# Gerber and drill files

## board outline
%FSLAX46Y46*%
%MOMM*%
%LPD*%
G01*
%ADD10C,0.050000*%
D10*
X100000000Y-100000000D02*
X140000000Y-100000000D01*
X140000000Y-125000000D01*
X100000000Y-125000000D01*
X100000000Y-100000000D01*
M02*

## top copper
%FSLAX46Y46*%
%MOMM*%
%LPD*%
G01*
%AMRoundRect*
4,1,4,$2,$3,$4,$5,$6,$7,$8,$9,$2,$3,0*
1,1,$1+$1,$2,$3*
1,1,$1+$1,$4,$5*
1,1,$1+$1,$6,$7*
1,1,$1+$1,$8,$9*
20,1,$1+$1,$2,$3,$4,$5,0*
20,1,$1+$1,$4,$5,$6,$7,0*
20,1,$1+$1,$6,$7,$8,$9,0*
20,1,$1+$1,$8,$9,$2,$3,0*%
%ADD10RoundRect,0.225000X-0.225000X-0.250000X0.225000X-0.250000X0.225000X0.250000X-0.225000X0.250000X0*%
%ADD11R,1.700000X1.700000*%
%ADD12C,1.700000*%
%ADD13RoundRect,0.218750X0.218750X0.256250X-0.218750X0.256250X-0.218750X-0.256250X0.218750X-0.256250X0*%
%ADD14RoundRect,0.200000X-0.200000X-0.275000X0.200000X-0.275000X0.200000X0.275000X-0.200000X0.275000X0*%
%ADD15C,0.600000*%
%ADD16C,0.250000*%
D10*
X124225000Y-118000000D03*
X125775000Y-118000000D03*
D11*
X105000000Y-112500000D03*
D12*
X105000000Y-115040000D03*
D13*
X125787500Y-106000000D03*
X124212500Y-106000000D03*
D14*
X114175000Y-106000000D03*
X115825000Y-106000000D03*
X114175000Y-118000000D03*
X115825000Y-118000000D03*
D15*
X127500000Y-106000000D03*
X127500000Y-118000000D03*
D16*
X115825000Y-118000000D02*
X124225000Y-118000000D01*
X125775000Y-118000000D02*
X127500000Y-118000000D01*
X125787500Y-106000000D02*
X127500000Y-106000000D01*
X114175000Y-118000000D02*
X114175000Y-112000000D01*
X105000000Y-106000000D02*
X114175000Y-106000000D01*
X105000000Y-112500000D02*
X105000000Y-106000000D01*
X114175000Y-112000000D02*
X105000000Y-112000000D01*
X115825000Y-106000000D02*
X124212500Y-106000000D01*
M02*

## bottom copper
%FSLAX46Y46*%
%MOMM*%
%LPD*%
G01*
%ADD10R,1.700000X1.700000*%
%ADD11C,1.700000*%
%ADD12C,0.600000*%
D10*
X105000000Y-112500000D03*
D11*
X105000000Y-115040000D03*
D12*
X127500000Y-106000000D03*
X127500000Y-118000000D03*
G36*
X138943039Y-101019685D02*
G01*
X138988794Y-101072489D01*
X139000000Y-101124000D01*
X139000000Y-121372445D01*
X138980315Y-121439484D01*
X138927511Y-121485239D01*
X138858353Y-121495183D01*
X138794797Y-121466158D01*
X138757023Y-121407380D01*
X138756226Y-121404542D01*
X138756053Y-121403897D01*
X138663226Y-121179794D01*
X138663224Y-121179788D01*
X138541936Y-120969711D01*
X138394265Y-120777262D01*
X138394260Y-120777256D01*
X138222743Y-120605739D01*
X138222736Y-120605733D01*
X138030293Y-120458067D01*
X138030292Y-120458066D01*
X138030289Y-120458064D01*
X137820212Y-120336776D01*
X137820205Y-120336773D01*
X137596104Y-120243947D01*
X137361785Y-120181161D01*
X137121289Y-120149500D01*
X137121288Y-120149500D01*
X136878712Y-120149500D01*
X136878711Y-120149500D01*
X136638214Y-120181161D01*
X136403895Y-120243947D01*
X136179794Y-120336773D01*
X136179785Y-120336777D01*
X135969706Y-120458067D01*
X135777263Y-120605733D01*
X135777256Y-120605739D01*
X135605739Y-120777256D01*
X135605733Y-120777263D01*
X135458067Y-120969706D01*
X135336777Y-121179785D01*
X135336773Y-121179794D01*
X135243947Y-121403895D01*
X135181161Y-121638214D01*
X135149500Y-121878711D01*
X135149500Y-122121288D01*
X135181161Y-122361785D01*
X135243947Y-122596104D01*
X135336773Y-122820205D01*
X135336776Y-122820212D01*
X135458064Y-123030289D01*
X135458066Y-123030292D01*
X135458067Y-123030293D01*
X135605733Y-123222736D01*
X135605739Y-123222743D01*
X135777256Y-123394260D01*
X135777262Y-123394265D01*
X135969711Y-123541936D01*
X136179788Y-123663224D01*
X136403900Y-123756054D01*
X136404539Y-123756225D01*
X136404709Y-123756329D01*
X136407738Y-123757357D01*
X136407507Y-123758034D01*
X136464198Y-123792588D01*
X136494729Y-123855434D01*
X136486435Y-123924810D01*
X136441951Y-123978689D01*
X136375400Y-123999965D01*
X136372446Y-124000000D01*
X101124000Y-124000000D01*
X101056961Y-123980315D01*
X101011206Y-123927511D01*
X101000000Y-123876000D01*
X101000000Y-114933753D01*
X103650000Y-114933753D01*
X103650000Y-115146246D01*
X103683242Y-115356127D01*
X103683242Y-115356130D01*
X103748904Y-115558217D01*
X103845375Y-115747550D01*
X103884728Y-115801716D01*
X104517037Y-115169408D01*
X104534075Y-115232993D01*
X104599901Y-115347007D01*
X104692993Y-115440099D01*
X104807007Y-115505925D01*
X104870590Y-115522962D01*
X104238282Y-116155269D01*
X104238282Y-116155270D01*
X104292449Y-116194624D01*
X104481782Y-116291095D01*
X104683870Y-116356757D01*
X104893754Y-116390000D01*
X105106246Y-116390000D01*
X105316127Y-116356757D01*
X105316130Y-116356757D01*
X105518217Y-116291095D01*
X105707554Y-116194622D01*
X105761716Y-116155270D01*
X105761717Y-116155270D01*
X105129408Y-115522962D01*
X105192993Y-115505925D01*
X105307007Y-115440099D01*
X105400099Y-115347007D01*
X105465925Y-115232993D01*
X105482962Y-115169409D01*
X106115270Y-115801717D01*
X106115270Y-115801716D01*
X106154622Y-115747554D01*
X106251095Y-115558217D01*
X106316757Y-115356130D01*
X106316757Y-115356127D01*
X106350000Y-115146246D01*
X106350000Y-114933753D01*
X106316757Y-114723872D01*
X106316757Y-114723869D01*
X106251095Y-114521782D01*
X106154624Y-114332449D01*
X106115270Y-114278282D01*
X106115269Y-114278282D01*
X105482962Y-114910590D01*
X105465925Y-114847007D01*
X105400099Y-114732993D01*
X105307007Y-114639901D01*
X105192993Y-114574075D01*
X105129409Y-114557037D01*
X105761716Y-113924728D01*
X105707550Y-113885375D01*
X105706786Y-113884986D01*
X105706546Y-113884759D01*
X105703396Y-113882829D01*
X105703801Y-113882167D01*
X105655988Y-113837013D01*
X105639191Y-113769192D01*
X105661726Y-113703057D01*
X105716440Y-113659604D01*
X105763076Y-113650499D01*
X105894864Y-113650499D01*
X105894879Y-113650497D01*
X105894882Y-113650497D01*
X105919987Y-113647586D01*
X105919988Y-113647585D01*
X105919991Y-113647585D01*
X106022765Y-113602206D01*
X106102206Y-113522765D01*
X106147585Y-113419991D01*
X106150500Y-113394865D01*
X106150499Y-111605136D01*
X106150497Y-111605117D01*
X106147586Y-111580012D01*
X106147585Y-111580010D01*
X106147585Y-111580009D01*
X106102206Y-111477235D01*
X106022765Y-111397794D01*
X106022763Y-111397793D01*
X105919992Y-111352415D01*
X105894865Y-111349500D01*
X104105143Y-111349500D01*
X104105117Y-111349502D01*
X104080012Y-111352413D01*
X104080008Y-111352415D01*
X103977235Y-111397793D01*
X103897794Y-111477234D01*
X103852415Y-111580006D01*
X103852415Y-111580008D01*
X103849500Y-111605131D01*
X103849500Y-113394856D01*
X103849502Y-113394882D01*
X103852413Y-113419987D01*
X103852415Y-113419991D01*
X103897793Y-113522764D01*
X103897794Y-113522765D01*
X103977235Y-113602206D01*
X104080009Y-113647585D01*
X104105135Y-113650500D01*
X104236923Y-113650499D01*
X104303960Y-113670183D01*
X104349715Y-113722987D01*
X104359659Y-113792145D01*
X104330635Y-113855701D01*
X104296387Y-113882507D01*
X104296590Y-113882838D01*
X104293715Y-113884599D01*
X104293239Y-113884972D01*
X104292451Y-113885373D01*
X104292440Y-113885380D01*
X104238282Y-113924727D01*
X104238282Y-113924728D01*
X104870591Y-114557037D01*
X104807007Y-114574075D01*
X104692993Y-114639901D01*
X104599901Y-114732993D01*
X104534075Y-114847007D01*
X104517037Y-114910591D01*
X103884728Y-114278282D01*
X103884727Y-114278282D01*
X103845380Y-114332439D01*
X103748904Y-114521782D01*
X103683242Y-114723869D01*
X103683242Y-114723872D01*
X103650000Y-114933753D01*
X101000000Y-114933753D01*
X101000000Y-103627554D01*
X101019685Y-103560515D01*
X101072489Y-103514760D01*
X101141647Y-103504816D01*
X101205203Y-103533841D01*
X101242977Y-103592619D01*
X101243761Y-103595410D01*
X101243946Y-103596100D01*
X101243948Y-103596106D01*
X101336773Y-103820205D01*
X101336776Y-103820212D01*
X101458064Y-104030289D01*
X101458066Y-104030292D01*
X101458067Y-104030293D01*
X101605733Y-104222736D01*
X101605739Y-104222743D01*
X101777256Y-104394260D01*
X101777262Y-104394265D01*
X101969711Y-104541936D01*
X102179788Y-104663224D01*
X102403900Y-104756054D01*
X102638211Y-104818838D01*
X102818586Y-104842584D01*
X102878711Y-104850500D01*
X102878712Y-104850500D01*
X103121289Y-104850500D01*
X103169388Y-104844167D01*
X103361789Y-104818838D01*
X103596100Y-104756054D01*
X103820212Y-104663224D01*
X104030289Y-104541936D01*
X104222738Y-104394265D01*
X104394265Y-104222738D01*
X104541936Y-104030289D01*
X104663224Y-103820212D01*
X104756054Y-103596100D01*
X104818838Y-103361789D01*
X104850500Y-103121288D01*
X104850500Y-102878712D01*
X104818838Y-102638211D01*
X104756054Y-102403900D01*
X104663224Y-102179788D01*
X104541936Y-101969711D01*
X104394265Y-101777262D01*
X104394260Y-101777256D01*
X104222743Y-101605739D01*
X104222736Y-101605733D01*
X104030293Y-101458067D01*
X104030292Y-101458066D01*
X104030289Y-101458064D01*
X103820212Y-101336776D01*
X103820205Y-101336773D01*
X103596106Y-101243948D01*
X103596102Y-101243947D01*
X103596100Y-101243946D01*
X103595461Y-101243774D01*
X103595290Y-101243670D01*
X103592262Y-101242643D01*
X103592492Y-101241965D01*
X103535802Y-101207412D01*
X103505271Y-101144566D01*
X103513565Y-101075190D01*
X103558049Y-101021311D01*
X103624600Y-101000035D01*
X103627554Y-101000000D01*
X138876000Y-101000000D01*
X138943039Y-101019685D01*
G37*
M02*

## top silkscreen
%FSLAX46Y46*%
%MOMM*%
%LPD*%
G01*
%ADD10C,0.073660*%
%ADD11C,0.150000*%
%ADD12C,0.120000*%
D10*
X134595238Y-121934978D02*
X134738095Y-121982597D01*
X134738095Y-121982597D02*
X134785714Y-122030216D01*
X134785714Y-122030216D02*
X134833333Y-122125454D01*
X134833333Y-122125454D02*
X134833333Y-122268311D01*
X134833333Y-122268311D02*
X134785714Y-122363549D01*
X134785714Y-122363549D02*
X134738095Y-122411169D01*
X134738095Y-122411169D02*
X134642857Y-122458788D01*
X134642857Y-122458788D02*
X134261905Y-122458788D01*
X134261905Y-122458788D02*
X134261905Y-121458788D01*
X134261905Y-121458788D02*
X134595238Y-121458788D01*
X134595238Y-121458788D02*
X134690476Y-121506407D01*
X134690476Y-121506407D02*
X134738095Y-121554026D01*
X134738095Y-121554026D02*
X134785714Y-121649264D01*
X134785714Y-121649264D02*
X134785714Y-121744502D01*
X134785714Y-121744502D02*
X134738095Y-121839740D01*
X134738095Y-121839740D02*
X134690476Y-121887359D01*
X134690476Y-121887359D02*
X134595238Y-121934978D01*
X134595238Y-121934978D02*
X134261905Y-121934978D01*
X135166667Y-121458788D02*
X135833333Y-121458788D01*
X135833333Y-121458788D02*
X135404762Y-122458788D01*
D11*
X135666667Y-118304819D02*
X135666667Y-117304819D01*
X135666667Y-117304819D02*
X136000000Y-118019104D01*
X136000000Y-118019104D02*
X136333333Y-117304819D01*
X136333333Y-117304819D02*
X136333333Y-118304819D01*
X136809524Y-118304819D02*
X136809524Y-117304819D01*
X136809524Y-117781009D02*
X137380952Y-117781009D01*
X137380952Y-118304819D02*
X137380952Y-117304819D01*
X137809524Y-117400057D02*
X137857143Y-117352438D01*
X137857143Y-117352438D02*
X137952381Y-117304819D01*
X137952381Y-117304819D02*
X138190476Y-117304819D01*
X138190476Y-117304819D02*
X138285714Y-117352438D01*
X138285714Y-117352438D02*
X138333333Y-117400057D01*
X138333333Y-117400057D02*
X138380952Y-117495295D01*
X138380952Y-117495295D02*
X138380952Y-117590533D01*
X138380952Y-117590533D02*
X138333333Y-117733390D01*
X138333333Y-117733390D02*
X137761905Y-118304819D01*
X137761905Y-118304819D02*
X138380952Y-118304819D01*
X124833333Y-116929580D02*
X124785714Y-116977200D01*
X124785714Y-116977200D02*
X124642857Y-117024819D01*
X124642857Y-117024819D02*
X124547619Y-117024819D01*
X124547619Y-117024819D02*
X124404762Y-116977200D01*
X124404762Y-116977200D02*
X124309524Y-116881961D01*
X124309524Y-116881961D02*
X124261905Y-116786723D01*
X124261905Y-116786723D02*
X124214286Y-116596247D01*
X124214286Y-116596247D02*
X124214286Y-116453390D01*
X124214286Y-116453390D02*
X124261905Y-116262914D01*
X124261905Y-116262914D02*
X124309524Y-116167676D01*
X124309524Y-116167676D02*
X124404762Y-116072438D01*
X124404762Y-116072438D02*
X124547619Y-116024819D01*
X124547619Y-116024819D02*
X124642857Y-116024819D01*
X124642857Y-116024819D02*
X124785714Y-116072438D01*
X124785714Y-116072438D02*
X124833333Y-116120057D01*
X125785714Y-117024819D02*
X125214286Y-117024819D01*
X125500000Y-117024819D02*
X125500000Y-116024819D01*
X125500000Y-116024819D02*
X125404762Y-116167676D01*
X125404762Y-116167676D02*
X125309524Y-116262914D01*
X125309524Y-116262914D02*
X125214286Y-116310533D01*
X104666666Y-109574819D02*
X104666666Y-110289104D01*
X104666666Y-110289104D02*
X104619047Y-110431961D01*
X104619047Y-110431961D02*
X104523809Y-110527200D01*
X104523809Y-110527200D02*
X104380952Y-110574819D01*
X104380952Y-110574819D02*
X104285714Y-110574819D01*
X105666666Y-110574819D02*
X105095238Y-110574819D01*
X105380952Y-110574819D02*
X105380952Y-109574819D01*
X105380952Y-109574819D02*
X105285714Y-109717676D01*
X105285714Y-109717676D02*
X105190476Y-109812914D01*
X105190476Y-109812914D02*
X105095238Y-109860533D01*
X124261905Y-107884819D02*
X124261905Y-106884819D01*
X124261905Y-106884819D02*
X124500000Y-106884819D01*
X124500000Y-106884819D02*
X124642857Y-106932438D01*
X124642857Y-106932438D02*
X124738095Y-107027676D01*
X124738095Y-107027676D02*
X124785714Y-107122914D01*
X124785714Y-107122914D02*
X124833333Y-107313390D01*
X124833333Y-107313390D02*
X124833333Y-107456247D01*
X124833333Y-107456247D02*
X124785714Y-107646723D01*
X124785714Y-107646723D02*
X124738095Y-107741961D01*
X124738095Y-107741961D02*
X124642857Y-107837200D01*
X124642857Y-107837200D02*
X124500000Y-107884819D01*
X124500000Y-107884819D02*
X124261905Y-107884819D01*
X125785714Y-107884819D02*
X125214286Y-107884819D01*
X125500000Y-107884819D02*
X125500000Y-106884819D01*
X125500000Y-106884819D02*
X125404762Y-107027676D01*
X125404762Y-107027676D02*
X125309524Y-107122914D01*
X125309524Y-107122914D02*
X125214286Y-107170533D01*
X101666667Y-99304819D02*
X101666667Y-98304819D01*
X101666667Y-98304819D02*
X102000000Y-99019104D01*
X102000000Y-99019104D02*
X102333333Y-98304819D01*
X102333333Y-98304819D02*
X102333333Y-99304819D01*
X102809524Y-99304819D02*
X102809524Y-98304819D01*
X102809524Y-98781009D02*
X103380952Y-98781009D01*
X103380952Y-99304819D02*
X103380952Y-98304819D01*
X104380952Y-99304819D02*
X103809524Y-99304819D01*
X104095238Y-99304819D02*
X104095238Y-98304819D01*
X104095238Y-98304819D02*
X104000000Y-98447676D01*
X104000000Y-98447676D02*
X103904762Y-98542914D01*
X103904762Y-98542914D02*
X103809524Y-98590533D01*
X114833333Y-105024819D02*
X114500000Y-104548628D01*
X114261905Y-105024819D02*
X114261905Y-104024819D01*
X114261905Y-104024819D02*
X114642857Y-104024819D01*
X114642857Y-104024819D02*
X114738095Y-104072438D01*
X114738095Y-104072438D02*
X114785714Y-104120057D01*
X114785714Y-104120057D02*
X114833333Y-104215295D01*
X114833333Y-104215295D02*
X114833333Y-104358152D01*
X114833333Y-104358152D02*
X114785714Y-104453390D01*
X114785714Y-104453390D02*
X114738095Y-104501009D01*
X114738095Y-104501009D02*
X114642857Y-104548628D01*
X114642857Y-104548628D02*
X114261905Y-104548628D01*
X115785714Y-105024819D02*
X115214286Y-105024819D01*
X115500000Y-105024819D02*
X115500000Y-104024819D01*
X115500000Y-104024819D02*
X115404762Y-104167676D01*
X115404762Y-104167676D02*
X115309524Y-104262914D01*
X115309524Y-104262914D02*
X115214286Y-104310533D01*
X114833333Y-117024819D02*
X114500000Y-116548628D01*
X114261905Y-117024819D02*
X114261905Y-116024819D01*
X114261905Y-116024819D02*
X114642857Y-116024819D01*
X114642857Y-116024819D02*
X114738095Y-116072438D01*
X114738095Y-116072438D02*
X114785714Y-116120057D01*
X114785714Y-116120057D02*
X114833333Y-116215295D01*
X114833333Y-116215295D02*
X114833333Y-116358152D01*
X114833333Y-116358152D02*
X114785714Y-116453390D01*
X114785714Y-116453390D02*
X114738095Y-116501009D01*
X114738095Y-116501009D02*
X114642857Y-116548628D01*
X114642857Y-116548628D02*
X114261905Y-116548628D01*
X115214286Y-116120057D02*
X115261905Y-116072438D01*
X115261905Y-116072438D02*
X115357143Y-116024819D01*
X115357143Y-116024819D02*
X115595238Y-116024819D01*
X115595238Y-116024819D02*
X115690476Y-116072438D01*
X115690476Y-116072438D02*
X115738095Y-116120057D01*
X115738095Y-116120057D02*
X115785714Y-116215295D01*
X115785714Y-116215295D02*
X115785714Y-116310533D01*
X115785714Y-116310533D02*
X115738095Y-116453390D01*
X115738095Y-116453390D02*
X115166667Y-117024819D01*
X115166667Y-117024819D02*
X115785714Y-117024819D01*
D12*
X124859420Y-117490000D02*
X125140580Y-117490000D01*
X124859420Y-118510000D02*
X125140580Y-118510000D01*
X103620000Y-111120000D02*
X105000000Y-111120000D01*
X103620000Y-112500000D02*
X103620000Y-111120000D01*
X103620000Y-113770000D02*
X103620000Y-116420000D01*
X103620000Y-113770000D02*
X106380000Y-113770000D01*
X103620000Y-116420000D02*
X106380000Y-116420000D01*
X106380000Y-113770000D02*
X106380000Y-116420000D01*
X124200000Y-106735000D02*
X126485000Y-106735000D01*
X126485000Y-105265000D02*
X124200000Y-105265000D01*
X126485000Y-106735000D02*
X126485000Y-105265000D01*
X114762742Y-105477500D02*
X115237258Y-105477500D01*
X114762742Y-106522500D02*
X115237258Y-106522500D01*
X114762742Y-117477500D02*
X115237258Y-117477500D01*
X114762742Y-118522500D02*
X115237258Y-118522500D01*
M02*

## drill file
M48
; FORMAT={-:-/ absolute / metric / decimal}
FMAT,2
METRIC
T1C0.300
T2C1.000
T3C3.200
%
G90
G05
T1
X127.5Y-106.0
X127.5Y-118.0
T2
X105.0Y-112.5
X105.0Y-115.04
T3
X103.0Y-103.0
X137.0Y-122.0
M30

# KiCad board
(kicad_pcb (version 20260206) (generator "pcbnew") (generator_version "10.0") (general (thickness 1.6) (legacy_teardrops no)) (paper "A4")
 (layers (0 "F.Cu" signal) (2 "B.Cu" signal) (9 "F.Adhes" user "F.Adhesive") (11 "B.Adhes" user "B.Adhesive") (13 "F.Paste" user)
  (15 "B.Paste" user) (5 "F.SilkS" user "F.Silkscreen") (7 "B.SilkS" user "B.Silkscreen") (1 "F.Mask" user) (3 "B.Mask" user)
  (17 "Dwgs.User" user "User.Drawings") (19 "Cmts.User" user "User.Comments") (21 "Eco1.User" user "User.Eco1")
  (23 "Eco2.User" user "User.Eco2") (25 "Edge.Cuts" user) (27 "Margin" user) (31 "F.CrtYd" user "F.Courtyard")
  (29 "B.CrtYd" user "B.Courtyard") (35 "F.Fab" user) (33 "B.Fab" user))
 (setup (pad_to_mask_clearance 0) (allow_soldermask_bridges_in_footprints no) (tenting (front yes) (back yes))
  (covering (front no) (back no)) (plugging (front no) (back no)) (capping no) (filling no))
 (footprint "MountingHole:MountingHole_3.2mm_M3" (layer "F.Cu") (at 137 122)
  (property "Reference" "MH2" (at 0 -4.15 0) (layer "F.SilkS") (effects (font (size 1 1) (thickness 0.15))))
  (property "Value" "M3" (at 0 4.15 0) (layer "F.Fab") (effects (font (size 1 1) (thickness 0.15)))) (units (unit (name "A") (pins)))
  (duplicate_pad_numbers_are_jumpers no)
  (pad "" np_thru_hole circle (at 0 0) (size 3.2 3.2) (drill 3.2) (layers "*.Cu" "*.Mask")))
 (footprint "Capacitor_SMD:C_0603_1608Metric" (layer "F.Cu") (at 125 118)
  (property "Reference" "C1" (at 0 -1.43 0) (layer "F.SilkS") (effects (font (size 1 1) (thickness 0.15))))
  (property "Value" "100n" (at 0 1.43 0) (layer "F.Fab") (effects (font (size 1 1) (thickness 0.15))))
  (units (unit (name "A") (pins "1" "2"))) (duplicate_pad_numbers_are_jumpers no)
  (fp_line (start -0.14058 -0.51) (end 0.14058 -0.51) (stroke (width 0.12) (type solid)) (layer "F.SilkS"))
  (fp_line (start -0.14058 0.51) (end 0.14058 0.51) (stroke (width 0.12) (type solid)) (layer "F.SilkS"))
  (pad "1" smd roundrect (at -0.775 0) (size 0.9 0.95) (layers "F.Cu" "F.Mask" "F.Paste") (roundrect_rratio 0.25) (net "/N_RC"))
  (pad "2" smd roundrect (at 0.775 0) (size 0.9 0.95) (layers "F.Cu" "F.Mask" "F.Paste") (roundrect_rratio 0.25) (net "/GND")))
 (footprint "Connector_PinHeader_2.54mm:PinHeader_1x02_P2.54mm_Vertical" (layer "F.Cu") (at 105 112.5)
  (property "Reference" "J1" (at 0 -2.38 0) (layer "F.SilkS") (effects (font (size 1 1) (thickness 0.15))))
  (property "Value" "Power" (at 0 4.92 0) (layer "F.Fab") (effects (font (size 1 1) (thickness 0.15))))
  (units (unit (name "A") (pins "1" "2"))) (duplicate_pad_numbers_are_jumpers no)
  (fp_line (start -1.38 -1.38) (end 0 -1.38) (stroke (width 0.12) (type solid)) (layer "F.SilkS"))
  (fp_line (start -1.38 0) (end -1.38 -1.38) (stroke (width 0.12) (type solid)) (layer "F.SilkS"))
  (fp_line (start -1.38 1.27) (end -1.38 3.92) (stroke (width 0.12) (type solid)) (layer "F.SilkS"))
  (fp_line (start -1.38 1.27) (end 1.38 1.27) (stroke (width 0.12) (type solid)) (layer "F.SilkS"))
  (fp_line (start -1.38 3.92) (end 1.38 3.92) (stroke (width 0.12) (type solid)) (layer "F.SilkS"))
  (fp_line (start 1.38 1.27) (end 1.38 3.92) (stroke (width 0.12) (type solid)) (layer "F.SilkS"))
  (pad "1" thru_hole rect (at 0 0) (size 1.7 1.7) (drill 1) (layers "*.Cu" "*.Mask") (remove_unused_layers no) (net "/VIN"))
  (pad "2" thru_hole circle (at 0 2.54) (size 1.7 1.7) (drill 1) (layers "*.Cu" "*.Mask") (remove_unused_layers no) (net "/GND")))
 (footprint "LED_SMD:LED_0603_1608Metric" (layer "F.Cu") (at 125 106 180)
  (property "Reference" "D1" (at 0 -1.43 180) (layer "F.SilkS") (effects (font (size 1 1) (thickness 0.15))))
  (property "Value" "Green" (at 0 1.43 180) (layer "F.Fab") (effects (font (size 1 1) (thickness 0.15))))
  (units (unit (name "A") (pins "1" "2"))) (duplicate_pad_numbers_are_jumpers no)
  (fp_line (start 0.8 -0.735) (end -1.485 -0.735) (stroke (width 0.12) (type solid)) (layer "F.SilkS"))
  (fp_line (start -1.485 0.735) (end 0.8 0.735) (stroke (width 0.12) (type solid)) (layer "F.SilkS"))
  (fp_line (start -1.485 -0.735) (end -1.485 0.735) (stroke (width 0.12) (type solid)) (layer "F.SilkS"))
  (pad "1" smd roundrect (at -0.7875 0 180) (size 0.875 0.95) (layers "F.Cu" "F.Mask" "F.Paste") (roundrect_rratio 0.25) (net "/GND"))
  (pad "2" smd roundrect (at 0.7875 0 180) (size 0.875 0.95) (layers "F.Cu" "F.Mask" "F.Paste") (roundrect_rratio 0.25) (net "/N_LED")))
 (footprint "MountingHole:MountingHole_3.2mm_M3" (layer "F.Cu") (at 103 103)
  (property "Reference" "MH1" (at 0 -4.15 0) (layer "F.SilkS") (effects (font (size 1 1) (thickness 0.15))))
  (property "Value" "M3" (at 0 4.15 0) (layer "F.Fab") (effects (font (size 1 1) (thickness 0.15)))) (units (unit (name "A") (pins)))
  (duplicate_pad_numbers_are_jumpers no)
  (pad "" np_thru_hole circle (at 0 0) (size 3.2 3.2) (drill 3.2) (layers "*.Cu" "*.Mask")))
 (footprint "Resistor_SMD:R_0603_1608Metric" (layer "F.Cu") (at 115 106)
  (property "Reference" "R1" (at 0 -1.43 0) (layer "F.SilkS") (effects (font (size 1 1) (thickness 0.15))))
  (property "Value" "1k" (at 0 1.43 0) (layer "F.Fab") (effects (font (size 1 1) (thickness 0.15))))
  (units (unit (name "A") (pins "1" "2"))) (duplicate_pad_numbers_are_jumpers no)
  (fp_line (start -0.237258 -0.5225) (end 0.237258 -0.5225) (stroke (width 0.12) (type solid)) (layer "F.SilkS"))
  (fp_line (start -0.237258 0.5225) (end 0.237258 0.5225) (stroke (width 0.12) (type solid)) (layer "F.SilkS"))
  (pad "1" smd roundrect (at -0.825 0) (size 0.8 0.95) (layers "F.Cu" "F.Mask" "F.Paste") (roundrect_rratio 0.25) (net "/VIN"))
  (pad "2" smd roundrect (at 0.825 0) (size 0.8 0.95) (layers "F.Cu" "F.Mask" "F.Paste") (roundrect_rratio 0.25) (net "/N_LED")))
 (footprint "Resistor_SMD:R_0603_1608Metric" (layer "F.Cu") (at 115 118)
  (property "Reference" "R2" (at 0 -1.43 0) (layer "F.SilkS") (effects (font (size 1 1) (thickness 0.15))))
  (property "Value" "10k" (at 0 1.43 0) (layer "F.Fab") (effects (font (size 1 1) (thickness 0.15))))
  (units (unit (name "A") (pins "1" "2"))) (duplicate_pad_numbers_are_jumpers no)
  (fp_line (start -0.237258 -0.5225) (end 0.237258 -0.5225) (stroke (width 0.12) (type solid)) (layer "F.SilkS"))
  (fp_line (start -0.237258 0.5225) (end 0.237258 0.5225) (stroke (width 0.12) (type solid)) (layer "F.SilkS"))
  (pad "1" smd roundrect (at -0.825 0) (size 0.8 0.95) (layers "F.Cu" "F.Mask" "F.Paste") (roundrect_rratio 0.25) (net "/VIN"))
  (pad "2" smd roundrect (at 0.825 0) (size 0.8 0.95) (layers "F.Cu" "F.Mask" "F.Paste") (roundrect_rratio 0.25) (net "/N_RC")))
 (gr_rect (start 100 100) (end 140 125) (stroke (width 0.05) (type default)) (fill no) (layer "Edge.Cuts"))
 (segment (start 115.825 118) (end 124.225 118) (width 0.25) (layer "F.Cu") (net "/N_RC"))
 (segment (start 125.775 118) (end 127.5 118) (width 0.25) (layer "F.Cu") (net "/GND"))
 (segment (start 125.7875 106) (end 127.5 106) (width 0.25) (layer "F.Cu") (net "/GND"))
 (via (at 127.5 106) (size 0.6) (drill 0.3) (layers "F.Cu" "B.Cu") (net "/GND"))
 (via (at 127.5 118) (size 0.6) (drill 0.3) (layers "F.Cu" "B.Cu") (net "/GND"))
 (segment (start 114.175 118) (end 114.175 112) (width 0.25) (layer "F.Cu") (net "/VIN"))
 (segment (start 105 106) (end 114.175 106) (width 0.25) (layer "F.Cu") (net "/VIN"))
 (segment (start 105 112.5) (end 105 106) (width 0.25) (layer "F.Cu") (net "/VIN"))
 (segment (start 114.175 112) (end 105 112) (width 0.25) (layer "F.Cu") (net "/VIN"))
 (segment (start 115.825 106) (end 124.2125 106) (width 0.25) (layer "F.Cu") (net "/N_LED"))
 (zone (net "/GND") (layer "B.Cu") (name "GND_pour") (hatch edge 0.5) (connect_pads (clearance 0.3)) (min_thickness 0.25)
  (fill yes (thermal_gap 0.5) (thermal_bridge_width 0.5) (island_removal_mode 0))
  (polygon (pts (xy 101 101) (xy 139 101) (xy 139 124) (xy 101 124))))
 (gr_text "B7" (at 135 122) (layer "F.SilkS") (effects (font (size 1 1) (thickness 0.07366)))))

